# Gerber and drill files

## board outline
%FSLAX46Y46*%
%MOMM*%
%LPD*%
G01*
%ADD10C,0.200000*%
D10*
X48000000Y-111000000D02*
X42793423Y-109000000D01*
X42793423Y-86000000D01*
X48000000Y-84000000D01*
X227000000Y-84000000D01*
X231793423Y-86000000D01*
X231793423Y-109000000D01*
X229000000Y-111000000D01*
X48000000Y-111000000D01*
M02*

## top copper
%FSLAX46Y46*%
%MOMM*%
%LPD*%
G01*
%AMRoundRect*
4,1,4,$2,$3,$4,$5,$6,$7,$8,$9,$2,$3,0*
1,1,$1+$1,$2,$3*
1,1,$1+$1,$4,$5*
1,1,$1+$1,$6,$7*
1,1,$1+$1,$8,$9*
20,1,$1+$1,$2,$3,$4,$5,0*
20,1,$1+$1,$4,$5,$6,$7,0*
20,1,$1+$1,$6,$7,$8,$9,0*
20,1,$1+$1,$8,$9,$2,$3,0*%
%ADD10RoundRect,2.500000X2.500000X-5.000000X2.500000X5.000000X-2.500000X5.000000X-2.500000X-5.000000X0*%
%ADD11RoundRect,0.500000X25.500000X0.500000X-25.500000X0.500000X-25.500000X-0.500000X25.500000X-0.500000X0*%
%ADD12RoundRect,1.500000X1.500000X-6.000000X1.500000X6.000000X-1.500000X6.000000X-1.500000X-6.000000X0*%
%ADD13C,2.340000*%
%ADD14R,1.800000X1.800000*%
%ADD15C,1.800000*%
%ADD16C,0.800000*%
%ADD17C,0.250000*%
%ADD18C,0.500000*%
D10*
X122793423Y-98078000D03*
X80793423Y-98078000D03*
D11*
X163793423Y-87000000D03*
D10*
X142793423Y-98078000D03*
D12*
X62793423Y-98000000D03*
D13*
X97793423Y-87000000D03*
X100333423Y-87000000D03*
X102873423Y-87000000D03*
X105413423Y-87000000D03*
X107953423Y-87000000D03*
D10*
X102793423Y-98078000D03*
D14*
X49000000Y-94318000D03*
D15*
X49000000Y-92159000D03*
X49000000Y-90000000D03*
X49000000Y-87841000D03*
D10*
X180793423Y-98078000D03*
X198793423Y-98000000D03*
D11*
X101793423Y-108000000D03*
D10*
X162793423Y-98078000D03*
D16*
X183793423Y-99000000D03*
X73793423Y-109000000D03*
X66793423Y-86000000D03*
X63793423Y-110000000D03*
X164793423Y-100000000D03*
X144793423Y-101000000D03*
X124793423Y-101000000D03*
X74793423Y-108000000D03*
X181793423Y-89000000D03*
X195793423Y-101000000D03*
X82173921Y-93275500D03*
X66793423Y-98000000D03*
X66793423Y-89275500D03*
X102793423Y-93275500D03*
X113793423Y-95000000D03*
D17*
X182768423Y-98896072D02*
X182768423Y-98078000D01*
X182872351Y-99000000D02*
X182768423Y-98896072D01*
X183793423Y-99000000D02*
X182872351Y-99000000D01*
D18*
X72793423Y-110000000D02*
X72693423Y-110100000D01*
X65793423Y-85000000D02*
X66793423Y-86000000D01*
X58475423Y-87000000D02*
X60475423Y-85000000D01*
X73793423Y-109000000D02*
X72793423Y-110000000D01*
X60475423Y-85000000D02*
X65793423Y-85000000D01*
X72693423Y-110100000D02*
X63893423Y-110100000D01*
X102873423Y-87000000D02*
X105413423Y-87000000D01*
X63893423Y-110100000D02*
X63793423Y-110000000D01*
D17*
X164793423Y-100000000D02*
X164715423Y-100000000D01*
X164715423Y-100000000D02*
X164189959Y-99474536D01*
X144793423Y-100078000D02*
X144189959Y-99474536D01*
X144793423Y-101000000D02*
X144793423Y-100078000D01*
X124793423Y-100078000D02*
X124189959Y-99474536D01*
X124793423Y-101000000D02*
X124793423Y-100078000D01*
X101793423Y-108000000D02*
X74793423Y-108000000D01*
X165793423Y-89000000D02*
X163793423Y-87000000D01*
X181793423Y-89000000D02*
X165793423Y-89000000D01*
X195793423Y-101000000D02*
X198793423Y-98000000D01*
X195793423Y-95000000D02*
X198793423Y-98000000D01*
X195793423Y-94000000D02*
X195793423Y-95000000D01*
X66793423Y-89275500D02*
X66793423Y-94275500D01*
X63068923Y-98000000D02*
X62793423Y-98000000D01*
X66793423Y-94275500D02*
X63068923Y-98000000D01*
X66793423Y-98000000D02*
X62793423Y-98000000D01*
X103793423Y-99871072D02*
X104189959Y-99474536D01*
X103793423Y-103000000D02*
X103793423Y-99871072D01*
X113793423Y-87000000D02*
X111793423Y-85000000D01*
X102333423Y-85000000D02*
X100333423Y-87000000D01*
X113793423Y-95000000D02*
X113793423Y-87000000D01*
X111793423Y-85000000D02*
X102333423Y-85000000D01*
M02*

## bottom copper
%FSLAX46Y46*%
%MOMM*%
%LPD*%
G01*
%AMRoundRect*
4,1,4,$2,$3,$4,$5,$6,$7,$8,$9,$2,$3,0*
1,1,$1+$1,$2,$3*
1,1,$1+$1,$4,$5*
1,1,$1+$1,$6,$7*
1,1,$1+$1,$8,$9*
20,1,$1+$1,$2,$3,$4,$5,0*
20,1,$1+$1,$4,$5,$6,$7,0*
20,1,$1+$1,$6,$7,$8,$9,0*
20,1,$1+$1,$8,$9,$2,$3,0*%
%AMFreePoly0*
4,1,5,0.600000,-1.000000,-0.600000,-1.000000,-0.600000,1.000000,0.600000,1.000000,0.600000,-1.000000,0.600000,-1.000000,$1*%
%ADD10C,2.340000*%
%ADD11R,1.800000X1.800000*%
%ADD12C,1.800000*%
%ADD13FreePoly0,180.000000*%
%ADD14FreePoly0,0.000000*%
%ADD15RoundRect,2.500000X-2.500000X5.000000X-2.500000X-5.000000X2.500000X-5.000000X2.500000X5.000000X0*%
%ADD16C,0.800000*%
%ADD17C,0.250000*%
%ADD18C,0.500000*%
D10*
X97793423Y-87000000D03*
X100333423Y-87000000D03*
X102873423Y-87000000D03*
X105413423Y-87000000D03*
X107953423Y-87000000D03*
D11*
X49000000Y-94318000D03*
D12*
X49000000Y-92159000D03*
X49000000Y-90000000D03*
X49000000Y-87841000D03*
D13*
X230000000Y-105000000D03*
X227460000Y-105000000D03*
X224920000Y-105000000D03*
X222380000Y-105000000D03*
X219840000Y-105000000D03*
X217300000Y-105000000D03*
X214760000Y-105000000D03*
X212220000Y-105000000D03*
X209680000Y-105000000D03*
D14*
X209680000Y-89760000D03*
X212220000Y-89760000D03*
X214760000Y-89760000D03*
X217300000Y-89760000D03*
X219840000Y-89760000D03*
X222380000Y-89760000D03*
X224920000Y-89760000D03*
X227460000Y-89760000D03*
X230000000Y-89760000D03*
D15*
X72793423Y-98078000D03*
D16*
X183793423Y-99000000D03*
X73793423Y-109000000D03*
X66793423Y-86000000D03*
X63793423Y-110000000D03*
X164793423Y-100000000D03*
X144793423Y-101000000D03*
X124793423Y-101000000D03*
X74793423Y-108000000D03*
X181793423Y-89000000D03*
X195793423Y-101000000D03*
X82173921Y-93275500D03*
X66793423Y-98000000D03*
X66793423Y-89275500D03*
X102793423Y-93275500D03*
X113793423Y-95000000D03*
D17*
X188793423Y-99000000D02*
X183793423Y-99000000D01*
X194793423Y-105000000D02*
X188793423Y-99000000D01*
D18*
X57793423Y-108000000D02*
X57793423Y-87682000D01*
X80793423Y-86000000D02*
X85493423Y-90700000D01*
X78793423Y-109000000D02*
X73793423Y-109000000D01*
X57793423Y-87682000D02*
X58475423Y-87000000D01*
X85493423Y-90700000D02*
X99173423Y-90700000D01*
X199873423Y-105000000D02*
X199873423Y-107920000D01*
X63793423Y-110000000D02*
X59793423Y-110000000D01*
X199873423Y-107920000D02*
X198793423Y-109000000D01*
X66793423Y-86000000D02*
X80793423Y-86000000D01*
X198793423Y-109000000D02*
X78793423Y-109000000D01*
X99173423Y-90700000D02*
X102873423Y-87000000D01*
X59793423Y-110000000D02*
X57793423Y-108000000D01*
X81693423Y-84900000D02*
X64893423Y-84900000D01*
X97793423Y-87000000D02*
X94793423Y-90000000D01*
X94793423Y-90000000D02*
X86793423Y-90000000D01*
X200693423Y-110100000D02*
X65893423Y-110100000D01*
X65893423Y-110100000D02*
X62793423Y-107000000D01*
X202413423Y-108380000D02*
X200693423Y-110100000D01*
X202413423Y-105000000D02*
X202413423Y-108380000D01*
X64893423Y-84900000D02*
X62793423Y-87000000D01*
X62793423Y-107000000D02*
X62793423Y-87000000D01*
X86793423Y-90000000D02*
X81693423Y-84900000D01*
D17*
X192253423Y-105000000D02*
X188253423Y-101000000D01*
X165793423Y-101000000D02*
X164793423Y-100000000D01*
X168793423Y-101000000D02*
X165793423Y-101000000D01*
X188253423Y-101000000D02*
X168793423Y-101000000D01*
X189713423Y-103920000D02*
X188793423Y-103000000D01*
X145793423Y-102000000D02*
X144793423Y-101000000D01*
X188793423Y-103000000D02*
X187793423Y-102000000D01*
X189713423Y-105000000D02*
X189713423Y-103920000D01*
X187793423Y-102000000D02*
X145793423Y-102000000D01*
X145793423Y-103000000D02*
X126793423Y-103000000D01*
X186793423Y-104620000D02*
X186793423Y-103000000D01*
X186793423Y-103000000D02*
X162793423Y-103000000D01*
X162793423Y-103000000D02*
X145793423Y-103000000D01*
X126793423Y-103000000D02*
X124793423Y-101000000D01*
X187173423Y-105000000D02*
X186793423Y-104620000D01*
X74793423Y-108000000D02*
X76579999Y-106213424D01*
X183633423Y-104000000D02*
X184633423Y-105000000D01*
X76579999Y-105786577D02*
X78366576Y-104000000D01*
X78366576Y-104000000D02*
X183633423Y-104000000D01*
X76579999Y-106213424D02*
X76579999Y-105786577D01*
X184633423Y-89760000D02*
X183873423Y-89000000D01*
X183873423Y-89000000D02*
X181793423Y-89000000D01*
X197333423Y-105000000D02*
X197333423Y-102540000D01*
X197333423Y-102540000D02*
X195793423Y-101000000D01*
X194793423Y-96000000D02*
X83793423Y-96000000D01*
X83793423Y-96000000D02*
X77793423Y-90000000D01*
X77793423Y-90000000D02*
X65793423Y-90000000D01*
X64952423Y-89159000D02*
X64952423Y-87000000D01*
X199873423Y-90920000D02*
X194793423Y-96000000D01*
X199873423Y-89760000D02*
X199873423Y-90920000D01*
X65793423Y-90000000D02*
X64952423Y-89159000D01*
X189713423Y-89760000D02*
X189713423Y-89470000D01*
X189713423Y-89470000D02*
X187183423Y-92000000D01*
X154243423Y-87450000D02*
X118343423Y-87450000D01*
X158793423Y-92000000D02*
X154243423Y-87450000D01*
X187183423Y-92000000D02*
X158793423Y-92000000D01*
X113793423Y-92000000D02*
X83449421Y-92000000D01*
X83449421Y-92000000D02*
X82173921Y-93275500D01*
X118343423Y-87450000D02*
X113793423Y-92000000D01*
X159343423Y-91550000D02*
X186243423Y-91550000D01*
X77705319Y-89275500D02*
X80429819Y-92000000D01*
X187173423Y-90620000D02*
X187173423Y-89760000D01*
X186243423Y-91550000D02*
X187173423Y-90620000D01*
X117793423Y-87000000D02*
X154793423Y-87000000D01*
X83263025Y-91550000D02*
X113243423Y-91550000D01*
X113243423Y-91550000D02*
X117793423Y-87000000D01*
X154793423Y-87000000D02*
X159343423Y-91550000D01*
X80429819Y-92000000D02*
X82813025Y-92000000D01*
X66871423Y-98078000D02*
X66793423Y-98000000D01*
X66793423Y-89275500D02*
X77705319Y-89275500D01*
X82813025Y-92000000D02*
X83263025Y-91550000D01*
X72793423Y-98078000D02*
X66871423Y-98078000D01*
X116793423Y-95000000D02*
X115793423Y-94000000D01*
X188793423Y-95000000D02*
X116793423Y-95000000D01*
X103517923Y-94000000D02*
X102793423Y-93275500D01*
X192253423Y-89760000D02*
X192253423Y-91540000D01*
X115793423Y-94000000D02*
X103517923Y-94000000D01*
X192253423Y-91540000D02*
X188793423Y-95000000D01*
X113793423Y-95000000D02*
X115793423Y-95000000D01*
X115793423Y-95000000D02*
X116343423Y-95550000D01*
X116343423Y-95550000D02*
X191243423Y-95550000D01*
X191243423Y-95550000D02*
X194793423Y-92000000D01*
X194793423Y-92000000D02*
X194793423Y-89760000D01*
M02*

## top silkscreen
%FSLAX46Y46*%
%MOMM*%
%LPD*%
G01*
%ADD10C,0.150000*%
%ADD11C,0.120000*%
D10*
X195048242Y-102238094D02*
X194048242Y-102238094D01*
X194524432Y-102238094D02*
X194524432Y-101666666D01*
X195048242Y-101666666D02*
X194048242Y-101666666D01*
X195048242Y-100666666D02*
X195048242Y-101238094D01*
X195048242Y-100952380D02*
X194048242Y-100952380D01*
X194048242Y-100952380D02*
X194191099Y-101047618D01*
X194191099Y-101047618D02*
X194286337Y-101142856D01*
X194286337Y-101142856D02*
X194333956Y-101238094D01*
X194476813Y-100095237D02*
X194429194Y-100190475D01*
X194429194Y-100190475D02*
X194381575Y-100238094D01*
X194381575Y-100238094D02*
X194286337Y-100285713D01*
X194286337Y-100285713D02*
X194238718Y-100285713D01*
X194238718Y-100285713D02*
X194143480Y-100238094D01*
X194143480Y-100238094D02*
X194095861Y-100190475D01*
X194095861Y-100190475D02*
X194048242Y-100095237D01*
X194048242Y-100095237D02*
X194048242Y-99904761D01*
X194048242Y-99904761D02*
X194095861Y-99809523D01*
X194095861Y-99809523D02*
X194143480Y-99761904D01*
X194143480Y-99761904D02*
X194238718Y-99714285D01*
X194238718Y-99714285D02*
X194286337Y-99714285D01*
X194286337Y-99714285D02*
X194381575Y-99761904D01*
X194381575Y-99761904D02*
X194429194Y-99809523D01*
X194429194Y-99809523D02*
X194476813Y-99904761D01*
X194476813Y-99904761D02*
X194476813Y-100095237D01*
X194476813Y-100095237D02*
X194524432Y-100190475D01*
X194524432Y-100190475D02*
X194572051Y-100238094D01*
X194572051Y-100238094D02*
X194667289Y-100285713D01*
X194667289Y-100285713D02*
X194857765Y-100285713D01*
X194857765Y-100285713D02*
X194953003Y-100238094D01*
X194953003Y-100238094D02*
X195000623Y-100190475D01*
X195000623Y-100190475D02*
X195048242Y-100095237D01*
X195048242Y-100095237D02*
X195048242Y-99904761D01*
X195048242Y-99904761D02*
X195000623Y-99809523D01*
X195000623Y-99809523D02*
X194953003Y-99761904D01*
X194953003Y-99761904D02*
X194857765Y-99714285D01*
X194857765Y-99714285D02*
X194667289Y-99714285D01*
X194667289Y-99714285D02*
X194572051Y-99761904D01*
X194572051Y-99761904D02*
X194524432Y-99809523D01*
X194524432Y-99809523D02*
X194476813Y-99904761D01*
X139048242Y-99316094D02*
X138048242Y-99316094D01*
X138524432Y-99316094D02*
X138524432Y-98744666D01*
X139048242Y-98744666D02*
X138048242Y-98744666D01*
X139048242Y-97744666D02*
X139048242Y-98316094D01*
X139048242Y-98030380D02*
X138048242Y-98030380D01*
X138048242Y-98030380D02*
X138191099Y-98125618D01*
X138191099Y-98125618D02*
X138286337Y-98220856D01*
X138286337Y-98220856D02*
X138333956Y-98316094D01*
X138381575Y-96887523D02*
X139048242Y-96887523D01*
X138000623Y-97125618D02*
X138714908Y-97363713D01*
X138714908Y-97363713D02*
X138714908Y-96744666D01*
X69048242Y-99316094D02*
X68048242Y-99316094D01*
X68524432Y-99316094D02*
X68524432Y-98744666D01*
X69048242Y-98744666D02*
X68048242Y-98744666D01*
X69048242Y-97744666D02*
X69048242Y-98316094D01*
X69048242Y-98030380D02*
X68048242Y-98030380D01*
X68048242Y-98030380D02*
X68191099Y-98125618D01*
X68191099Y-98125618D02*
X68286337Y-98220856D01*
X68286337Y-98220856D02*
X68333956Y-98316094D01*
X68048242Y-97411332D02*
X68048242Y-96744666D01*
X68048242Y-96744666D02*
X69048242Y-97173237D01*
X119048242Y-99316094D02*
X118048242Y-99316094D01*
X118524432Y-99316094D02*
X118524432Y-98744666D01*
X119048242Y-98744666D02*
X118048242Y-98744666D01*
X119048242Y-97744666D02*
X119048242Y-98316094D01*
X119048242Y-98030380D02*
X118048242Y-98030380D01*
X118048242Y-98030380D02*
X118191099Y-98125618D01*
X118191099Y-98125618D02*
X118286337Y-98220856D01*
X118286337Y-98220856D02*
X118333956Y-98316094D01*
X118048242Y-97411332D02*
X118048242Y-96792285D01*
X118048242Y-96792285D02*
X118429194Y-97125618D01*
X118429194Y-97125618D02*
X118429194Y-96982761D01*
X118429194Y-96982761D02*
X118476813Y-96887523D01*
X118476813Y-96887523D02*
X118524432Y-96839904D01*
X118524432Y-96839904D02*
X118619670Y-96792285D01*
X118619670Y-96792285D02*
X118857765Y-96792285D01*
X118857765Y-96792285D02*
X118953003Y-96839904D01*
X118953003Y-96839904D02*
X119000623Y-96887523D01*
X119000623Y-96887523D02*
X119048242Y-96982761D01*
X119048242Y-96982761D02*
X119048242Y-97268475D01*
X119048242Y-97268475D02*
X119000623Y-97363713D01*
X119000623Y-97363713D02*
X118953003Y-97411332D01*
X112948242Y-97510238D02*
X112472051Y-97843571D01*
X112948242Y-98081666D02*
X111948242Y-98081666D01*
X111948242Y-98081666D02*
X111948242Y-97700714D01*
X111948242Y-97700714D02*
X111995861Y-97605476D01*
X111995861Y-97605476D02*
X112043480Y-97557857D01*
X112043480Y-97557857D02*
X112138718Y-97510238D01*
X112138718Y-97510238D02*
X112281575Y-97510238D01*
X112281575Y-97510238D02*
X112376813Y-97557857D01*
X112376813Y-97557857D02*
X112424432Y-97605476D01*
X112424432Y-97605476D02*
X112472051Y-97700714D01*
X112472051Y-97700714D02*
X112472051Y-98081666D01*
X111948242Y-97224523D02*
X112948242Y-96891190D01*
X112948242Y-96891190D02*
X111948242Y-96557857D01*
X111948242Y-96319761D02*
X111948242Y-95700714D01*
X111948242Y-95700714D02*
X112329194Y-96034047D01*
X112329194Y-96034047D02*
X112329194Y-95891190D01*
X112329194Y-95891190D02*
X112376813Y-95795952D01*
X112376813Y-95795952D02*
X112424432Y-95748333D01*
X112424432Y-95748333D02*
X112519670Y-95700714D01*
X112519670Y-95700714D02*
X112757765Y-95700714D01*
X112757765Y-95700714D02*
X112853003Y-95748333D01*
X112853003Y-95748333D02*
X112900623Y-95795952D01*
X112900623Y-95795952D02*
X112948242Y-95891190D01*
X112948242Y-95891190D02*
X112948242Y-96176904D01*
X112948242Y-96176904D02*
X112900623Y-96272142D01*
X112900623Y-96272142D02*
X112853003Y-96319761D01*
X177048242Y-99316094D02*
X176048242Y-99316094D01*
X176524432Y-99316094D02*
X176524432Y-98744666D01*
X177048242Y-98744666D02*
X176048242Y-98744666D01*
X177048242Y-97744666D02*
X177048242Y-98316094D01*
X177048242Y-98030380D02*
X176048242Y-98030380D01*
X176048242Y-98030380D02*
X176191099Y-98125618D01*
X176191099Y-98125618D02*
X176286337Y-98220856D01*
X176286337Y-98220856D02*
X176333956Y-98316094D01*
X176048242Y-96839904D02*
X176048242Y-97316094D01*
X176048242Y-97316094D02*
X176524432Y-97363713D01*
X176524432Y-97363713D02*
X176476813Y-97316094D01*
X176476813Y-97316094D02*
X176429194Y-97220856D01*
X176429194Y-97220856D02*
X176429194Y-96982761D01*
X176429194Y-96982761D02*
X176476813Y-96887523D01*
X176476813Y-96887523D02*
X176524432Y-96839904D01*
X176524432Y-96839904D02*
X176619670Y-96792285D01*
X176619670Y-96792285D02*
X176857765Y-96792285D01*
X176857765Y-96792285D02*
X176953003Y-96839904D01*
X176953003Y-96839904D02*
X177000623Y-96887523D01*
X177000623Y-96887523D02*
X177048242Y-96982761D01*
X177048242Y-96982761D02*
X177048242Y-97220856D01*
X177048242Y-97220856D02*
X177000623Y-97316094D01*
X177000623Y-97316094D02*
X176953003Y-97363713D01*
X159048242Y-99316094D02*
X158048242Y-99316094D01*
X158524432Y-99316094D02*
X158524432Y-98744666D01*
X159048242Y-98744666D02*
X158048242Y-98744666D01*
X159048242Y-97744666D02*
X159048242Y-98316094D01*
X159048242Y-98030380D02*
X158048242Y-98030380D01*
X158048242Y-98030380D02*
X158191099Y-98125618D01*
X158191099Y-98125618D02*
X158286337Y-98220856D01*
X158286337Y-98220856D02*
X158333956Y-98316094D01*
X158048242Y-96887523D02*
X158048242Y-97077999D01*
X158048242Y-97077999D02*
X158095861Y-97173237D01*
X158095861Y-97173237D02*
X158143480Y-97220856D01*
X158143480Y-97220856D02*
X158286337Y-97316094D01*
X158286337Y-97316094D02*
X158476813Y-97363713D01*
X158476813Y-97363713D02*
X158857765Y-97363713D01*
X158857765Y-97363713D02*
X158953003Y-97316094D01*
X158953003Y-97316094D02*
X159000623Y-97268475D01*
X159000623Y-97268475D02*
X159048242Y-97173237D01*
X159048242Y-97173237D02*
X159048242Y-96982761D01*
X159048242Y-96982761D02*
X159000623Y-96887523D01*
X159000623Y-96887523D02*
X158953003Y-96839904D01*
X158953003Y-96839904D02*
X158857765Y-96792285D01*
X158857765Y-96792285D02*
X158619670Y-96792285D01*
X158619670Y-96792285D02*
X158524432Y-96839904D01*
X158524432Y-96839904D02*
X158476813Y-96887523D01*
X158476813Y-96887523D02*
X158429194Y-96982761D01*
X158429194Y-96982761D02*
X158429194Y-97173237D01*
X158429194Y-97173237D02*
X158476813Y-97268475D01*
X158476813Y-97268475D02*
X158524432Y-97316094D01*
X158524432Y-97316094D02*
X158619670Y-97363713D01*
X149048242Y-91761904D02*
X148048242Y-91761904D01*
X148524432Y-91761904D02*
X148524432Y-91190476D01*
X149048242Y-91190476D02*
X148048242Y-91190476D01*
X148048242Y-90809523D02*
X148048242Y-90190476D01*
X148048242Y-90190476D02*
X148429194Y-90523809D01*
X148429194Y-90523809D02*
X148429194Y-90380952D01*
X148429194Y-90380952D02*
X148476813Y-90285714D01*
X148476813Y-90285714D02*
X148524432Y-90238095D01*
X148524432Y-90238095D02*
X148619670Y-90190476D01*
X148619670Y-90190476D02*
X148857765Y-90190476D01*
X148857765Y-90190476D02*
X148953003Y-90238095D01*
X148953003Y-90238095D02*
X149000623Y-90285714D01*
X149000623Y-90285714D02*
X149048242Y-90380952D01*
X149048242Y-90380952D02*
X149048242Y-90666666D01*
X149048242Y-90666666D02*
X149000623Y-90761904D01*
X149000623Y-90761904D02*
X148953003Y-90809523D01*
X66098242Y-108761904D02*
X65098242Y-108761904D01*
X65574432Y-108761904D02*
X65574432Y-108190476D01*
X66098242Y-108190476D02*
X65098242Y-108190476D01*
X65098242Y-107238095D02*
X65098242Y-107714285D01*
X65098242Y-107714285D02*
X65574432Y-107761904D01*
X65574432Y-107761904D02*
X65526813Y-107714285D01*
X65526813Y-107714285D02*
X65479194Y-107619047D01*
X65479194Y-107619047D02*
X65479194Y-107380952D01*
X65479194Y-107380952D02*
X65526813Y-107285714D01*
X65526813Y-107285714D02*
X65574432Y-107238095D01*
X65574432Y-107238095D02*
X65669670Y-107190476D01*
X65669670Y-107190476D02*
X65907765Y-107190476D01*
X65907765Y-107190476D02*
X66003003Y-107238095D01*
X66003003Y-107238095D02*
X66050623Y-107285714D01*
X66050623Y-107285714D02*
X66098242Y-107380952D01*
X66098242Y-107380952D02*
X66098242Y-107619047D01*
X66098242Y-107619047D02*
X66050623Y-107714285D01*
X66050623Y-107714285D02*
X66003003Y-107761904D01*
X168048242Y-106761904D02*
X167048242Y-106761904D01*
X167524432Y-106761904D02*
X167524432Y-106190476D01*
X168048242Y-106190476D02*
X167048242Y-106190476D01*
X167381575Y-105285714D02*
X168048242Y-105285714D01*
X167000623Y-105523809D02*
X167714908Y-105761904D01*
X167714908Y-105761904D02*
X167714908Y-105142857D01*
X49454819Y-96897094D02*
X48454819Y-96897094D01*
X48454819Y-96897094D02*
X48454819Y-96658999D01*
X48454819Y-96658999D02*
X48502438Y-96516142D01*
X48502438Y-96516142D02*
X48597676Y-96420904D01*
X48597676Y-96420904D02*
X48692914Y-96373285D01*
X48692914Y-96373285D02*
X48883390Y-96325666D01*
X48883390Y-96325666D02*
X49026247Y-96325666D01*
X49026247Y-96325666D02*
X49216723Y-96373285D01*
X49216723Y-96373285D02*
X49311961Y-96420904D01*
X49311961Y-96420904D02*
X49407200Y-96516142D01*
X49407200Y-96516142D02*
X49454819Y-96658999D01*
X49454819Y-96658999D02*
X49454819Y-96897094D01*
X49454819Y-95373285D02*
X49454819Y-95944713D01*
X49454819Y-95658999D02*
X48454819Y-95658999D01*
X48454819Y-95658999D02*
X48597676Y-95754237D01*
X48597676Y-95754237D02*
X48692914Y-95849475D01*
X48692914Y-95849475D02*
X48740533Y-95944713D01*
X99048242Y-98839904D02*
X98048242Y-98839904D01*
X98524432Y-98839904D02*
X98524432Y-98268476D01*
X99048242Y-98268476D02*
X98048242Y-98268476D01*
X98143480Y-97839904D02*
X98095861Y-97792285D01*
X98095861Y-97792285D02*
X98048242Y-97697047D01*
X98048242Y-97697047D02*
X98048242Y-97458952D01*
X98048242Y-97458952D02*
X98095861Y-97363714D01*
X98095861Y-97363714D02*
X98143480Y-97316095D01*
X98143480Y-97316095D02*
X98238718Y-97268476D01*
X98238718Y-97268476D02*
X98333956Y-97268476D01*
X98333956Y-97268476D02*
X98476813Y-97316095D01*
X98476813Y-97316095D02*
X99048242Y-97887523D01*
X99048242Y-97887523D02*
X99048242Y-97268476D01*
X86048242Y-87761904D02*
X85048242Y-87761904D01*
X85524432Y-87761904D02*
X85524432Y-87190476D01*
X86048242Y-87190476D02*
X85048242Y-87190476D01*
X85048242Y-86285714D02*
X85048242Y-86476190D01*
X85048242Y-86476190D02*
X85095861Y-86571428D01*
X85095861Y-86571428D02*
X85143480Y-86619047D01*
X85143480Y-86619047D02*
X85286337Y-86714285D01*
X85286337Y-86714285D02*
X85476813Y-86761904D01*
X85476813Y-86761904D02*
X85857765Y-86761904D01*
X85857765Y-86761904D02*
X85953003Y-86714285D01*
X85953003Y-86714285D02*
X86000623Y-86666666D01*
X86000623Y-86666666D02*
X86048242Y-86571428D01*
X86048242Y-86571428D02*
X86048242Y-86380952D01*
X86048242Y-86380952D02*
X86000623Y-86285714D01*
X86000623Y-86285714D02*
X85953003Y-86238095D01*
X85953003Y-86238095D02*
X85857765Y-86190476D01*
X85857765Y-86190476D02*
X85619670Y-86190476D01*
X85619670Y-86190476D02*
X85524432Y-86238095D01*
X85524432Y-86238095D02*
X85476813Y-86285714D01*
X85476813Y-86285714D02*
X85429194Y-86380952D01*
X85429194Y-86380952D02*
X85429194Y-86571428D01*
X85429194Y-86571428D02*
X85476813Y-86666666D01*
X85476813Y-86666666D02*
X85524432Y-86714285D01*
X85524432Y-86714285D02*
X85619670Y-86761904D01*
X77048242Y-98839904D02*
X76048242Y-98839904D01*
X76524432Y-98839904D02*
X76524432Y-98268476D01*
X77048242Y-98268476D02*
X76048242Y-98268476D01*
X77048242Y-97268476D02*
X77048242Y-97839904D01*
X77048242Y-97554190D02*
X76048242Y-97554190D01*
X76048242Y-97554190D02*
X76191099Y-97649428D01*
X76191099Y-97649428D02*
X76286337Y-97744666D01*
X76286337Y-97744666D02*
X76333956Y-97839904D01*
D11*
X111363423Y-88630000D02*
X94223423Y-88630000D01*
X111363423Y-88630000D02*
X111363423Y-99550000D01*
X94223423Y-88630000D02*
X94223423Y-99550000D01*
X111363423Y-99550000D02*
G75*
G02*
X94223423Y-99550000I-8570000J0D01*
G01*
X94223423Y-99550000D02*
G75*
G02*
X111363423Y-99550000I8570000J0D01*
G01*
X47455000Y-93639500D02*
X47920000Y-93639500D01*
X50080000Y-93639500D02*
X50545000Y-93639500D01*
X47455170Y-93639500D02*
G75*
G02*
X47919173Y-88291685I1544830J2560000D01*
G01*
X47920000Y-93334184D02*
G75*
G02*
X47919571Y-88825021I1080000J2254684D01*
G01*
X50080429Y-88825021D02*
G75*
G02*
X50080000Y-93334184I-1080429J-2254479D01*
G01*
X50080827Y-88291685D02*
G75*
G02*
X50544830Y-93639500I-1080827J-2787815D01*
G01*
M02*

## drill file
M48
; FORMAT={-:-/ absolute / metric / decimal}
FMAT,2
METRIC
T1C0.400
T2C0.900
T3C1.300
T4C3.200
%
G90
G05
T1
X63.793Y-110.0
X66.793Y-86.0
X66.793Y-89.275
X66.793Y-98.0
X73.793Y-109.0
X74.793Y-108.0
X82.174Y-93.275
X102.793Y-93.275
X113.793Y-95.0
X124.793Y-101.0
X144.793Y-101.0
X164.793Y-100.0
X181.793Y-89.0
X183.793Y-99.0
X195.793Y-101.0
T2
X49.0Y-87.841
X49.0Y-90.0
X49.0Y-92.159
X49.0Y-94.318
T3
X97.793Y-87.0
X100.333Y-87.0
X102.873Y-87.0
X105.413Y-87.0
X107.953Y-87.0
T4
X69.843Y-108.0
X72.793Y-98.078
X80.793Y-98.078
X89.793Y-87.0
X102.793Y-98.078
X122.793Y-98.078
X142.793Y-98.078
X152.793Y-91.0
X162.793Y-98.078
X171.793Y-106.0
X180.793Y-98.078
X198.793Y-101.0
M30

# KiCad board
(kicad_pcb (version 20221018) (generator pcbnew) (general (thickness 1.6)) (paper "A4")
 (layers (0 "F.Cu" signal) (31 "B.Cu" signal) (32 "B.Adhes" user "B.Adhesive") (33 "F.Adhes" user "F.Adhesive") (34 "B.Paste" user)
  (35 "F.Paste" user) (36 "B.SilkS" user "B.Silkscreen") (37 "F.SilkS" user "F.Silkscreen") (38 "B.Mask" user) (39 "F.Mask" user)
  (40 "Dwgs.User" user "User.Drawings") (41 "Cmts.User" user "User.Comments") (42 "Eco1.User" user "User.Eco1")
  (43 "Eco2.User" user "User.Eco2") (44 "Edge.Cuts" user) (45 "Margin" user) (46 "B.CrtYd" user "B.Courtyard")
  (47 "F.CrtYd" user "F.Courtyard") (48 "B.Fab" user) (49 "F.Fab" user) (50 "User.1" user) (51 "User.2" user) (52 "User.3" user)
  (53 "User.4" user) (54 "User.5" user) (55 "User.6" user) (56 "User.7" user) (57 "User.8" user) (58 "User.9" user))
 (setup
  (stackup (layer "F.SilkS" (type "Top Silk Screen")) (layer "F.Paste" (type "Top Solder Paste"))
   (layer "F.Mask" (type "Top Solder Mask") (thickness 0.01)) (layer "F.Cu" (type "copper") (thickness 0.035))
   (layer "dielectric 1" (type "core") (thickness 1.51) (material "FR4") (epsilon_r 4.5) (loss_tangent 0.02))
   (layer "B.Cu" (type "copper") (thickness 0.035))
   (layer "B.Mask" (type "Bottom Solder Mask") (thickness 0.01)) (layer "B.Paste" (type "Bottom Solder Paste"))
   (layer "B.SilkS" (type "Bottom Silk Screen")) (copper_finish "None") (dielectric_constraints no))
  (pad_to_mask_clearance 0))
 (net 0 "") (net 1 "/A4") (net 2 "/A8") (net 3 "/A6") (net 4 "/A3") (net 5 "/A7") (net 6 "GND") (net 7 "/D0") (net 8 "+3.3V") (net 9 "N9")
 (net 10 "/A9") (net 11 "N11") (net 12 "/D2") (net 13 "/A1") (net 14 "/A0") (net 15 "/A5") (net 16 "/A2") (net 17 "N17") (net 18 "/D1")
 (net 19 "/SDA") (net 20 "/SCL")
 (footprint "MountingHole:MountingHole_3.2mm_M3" (layer "F.Cu") (at 198.793423 101 90)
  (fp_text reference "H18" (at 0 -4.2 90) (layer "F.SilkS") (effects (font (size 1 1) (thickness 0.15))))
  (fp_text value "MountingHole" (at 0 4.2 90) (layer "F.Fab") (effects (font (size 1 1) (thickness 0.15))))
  (pad "" np_thru_hole circle (at 0 0 90) (size 3.2 3.2) (drill 3.2) (layers "*.Cu" "*.Mask")))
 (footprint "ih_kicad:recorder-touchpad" (layer "F.Cu") (at 122.793423 98.078 90)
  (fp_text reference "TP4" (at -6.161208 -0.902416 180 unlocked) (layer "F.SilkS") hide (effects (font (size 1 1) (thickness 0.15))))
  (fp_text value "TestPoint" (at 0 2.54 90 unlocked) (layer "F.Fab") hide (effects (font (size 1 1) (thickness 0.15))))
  (pad "1" smd roundrect (at 0 0 90) (size 15 10) (layers "F.Cu" "F.Mask") (roundrect_rratio 0.25) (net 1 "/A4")))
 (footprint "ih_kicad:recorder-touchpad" (layer "F.Cu") (at 80.793423 98.078 90)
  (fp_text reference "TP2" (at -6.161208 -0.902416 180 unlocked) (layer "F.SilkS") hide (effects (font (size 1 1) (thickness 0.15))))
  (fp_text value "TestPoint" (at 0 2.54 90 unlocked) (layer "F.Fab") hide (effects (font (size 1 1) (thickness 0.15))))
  (pad "1" smd roundrect (at 0 0 90) (size 15 10) (layers "F.Cu" "F.Mask") (roundrect_rratio 0.25) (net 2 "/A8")))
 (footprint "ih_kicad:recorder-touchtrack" (layer "F.Cu") (at 163.793423 87 180)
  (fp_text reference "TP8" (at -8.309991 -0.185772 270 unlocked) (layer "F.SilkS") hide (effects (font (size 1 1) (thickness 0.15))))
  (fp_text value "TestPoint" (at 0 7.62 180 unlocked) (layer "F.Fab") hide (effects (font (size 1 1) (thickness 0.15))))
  (pad "1" smd roundrect (at 0 0 180) (size 52 2) (layers "F.Cu" "F.Mask") (roundrect_rratio 0.25) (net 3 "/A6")))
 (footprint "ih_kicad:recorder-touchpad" (layer "F.Cu") (at 142.793423 98.078 90)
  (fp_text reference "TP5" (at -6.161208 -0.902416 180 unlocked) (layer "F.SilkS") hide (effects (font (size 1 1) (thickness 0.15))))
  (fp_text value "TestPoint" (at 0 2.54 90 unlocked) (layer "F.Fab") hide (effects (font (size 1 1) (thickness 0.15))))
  (pad "1" smd roundrect (at 0 0 90) (size 15 10) (layers "F.Cu" "F.Mask") (roundrect_rratio 0.25) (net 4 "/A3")))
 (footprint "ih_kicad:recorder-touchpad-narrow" (layer "F.Cu") (at 62.793423 98 90)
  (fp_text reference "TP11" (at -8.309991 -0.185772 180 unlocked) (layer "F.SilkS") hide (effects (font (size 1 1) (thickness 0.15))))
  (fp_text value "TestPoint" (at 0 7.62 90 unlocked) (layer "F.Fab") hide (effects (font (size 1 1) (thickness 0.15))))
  (pad "1" smd roundrect (at 0 0 90) (size 15 6) (layers "F.Cu" "F.Mask") (roundrect_rratio 0.25) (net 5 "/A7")))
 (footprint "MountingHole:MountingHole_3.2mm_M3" (layer "F.Cu") (at 142.793423 98.078 90)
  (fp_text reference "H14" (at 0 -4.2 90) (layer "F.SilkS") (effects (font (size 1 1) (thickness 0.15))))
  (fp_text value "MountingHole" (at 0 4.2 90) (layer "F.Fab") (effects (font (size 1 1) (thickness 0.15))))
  (pad "" np_thru_hole circle (at 0 0 90) (size 3.2 3.2) (drill 3.2) (layers "*.Cu" "*.Mask")))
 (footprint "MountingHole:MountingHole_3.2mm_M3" (layer "F.Cu") (at 72.793423 98.078 90)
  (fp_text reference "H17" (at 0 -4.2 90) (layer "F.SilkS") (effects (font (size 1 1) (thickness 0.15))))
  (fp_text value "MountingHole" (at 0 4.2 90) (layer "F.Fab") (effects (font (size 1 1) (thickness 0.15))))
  (pad "" np_thru_hole circle (at 0 0 90) (size 3.2 3.2) (drill 3.2) (layers "*.Cu" "*.Mask")))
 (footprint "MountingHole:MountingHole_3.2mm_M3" (layer "F.Cu") (at 122.793423 98.078 90)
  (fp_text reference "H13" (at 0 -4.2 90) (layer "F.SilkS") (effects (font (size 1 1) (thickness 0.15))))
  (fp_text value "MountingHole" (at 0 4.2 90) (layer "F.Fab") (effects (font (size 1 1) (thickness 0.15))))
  (pad "" np_thru_hole circle (at 0 0 90) (size 3.2 3.2) (drill 3.2) (layers "*.Cu" "*.Mask")))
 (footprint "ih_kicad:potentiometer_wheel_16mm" (layer "F.Cu") (at 97.793423 87 -90)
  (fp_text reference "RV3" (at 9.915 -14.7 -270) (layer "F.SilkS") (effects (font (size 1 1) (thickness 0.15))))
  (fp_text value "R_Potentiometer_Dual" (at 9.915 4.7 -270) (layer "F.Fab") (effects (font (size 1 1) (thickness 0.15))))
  (fp_line (start 1.63 -13.57) (end 1.63 3.57) (stroke (width 0.12) (type solid)) (layer "F.SilkS"))
  (fp_line (start 1.63 -13.57) (end 12.55 -13.57) (stroke (width 0.12) (type solid)) (layer "F.SilkS"))
  (fp_line (start 1.63 3.57) (end 12.55 3.57) (stroke (width 0.12) (type solid)) (layer "F.SilkS"))
  (fp_circle (center 12.55 -5) (end 21.12 -5) (stroke (width 0.12) (type solid)) (fill none) (layer "F.SilkS"))
  (pad "1" thru_hole circle (at 0 0 270) (size 2.34 2.34) (drill 1.3) (layers "*.Cu" "*.Mask") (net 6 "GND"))
  (pad "2" thru_hole circle (at 0 -2.54 270) (size 2.34 2.34) (drill 1.3) (layers "*.Cu" "*.Mask") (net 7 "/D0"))
  (pad "3" thru_hole circle (at 0 -5.08 270) (size 2.34 2.34) (drill 1.3) (layers "*.Cu" "*.Mask") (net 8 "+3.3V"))
  (pad "4" thru_hole circle (at 0 -7.62 270) (size 2.34 2.34) (drill 1.3) (layers "*.Cu" "*.Mask") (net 8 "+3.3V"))
  (pad "5" thru_hole circle (at 0 -10.16 270) (size 2.34 2.34) (drill 1.3) (layers "*.Cu" "*.Mask") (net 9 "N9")))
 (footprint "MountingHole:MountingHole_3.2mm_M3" (layer "F.Cu") (at 180.793423 98.078 90)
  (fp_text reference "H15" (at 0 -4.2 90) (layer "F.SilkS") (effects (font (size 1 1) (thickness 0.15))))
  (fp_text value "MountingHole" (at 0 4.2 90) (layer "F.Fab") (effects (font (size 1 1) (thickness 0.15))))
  (pad "" np_thru_hole circle (at 0 0 90) (size 3.2 3.2) (drill 3.2) (layers "*.Cu" "*.Mask")))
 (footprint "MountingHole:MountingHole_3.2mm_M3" (layer "F.Cu") (at 162.793423 98.078 90)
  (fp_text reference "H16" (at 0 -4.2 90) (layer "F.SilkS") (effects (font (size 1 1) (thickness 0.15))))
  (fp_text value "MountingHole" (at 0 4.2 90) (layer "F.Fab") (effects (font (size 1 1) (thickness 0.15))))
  (pad "" np_thru_hole circle (at 0 0 90) (size 3.2 3.2) (drill 3.2) (layers "*.Cu" "*.Mask")))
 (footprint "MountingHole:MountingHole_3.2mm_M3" (layer "F.Cu") (at 152.793423 91 90)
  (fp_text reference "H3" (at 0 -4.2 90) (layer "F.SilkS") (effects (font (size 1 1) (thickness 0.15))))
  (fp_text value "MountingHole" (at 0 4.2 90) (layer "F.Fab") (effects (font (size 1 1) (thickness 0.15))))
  (pad "" np_thru_hole circle (at 0 0 90) (size 3.2 3.2) (drill 3.2) (layers "*.Cu" "*.Mask")))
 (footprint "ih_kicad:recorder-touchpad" (layer "F.Cu") (at 102.793423 98.078 90)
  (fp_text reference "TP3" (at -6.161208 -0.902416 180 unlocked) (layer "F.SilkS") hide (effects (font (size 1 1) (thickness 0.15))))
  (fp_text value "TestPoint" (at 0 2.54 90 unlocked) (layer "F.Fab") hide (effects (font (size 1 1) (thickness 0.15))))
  (pad "1" smd roundrect (at 0 0 90) (size 15 10) (layers "F.Cu" "F.Mask") (roundrect_rratio 0.25) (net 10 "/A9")))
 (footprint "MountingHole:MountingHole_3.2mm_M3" (layer "F.Cu") (at 69.843423 108 90)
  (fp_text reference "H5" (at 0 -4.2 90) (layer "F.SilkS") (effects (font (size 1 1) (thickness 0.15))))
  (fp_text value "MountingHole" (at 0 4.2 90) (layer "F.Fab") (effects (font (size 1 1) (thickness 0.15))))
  (pad "" np_thru_hole circle (at 0 0 90) (size 3.2 3.2) (drill 3.2) (layers "*.Cu" "*.Mask")))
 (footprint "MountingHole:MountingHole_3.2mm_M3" (layer "F.Cu") (at 171.793423 106 90)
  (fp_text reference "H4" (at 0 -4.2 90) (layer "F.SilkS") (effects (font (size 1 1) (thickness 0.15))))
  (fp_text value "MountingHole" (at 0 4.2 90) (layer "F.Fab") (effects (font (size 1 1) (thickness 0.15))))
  (pad "" np_thru_hole circle (at 0 0 90) (size 3.2 3.2) (drill 3.2) (layers "*.Cu" "*.Mask")))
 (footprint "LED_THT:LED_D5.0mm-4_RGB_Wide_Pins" (layer "F.Cu") (at 49 94.318 90)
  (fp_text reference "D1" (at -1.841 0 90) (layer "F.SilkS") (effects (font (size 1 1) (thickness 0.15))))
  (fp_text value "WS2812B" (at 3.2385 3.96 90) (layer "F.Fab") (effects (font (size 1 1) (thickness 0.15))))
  (fp_line (start 0.6785 -1.545) (end 0.6785 -1.08) (stroke (width 0.12) (type solid)) (layer "F.SilkS"))
  (fp_line (start 0.6785 1.08) (end 0.6785 1.545) (stroke (width 0.12) (type solid)) (layer "F.SilkS"))
  (fp_arc (start 0.6785 -1.54483) (mid 3.496956 -2.978809) (end 6.026315 -1.080827) (stroke (width 0.12) (type solid)) (layer "F.SilkS"))
  (fp_arc (start 0.983816 -1.08) (mid 3.238262 -2.5) (end 5.492979 -1.080429) (stroke (width 0.12) (type solid)) (layer "F.SilkS"))
  (fp_arc (start 5.492979 1.080429) (mid 3.238262 2.5) (end 0.983816 1.08) (stroke (width 0.12) (type solid)) (layer "F.SilkS"))
  (fp_arc (start 6.026315 1.080827) (mid 3.496956 2.978808) (end 0.6785 1.54483) (stroke (width 0.12) (type solid)) (layer "F.SilkS"))
  (pad "1" thru_hole rect (at 0 0 90) (size 1.8 1.8) (drill 0.9) (layers "*.Cu" "*.Mask") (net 8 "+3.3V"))
  (pad "2" thru_hole circle (at 2.159 0 90) (size 1.8 1.8) (drill 0.9) (layers "*.Cu" "*.Mask") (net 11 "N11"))
  (pad "3" thru_hole circle (at 4.318 0 90) (size 1.8 1.8) (drill 0.9) (layers "*.Cu" "*.Mask") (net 6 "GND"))
  (pad "4" thru_hole circle (at 6.477 0 90) (size 1.8 1.8) (drill 0.9) (layers "*.Cu" "*.Mask") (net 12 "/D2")))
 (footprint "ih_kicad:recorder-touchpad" (layer "F.Cu") (at 180.793423 98.078 90)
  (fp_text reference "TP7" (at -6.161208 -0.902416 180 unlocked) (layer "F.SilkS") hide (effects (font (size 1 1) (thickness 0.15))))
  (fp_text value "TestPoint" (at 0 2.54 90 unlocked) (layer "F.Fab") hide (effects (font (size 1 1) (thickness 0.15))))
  (pad "1" smd roundrect (at 0 0 90) (size 15 10) (layers "F.Cu" "F.Mask") (roundrect_rratio 0.25) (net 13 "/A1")))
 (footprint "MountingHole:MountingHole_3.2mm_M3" (layer "F.Cu") (at 102.793423 98.078 90)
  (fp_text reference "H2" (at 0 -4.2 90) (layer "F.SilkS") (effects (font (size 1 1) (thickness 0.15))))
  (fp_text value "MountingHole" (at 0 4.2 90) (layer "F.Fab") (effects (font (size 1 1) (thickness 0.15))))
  (pad "" np_thru_hole circle (at 0 0 90) (size 3.2 3.2) (drill 3.2) (layers "*.Cu" "*.Mask")))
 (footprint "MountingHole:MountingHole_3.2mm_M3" (layer "F.Cu") (at 89.793423 87 90)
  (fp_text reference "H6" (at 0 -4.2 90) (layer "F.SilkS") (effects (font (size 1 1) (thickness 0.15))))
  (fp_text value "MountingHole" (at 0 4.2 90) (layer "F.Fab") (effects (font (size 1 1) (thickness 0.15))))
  (pad "" np_thru_hole circle (at 0 0 90) (size 3.2 3.2) (drill 3.2) (layers "*.Cu" "*.Mask")))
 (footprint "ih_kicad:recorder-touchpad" (layer "F.Cu") (at 198.793423 98 90)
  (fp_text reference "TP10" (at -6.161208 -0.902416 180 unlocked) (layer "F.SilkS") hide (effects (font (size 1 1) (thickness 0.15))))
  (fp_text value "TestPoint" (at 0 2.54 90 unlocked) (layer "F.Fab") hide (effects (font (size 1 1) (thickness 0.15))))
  (pad "1" smd roundrect (at 0 0 90) (size 15 10) (layers "F.Cu" "F.Mask") (roundrect_rratio 0.25) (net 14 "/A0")))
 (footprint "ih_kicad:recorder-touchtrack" (layer "F.Cu") (at 101.793423 108 180)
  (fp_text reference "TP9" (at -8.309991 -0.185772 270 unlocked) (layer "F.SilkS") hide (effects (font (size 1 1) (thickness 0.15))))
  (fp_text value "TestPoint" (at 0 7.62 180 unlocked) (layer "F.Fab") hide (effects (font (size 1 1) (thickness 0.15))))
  (pad "1" smd roundrect (at 0 0 180) (size 52 2) (layers "F.Cu" "F.Mask") (roundrect_rratio 0.25) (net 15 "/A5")))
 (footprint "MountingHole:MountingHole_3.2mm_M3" (layer "F.Cu") (at 80.793423 98.078 90)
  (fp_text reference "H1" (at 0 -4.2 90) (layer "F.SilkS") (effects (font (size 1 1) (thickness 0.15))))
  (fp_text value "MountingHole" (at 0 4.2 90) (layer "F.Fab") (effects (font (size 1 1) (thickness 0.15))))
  (pad "" np_thru_hole circle (at 0 0 90) (size 3.2 3.2) (drill 3.2) (layers "*.Cu" "*.Mask")))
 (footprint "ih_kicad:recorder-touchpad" (layer "F.Cu") (at 162.793423 98.078 90)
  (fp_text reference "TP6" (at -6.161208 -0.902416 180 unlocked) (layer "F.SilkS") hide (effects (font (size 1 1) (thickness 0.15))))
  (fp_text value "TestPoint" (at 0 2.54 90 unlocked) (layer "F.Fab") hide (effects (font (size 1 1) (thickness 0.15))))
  (pad "1" smd roundrect (at 0 0 90) (size 15 10) (layers "F.Cu" "F.Mask") (roundrect_rratio 0.25) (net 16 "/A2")))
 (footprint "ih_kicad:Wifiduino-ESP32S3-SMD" (layer "B.Cu") (at 219.84 97.38 90)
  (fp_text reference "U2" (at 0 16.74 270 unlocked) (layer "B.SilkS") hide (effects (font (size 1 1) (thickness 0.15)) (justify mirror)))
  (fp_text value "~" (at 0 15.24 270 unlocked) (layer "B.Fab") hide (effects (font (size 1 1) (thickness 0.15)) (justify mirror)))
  (pad "1" smd custom (at -7.62 10.16 180) (size 1.2 2) (layers "B.Cu" "B.Paste" "B.Mask") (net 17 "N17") (thermal_bridge_angle 45)
   (options (clearance outline) (anchor rect)) (primitives))
  (pad "2" smd custom (at -7.62 7.62 180) (size 1.2 2) (layers "B.Cu" "B.Paste" "B.Mask") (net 6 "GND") (thermal_bridge_angle 45)
   (options (clearance outline) (anchor rect)) (primitives))
  (pad "3" smd custom (at -7.62 5.08 180) (size 1.2 2) (layers "B.Cu" "B.Paste" "B.Mask") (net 8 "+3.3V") (thermal_bridge_angle 45)
   (options (clearance outline) (anchor rect)) (primitives))
  (pad "4" smd custom (at -7.62 2.54 180) (size 1.2 2) (layers "B.Cu" "B.Paste" "B.Mask") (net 14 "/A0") (thermal_bridge_angle 45)
   (options (clearance outline) (anchor rect)) (primitives))
  (pad "5" smd custom (at -7.62 0 180) (size 1.2 2) (layers "B.Cu" "B.Paste" "B.Mask") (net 13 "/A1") (thermal_bridge_angle 45)
   (options (clearance outline) (anchor rect)) (primitives))
  (pad "6" smd custom (at -7.62 -2.54 180) (size 1.2 2) (layers "B.Cu" "B.Paste" "B.Mask") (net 16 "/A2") (thermal_bridge_angle 45)
   (options (clearance outline) (anchor rect)) (primitives))
  (pad "7" smd custom (at -7.62 -5.08 180) (size 1.2 2) (layers "B.Cu" "B.Paste" "B.Mask") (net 4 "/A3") (thermal_bridge_angle 45)
   (options (clearance outline) (anchor rect)) (primitives))
  (pad "8" smd custom (at -7.62 -7.62 180) (size 1.2 2) (layers "B.Cu" "B.Paste" "B.Mask") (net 1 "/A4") (thermal_bridge_angle 45)
   (options (clearance outline) (anchor rect)) (primitives))
  (pad "9" smd custom (at -7.62 -10.16 180) (size 1.2 2) (layers "B.Cu" "B.Paste" "B.Mask") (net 15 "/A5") (thermal_bridge_angle 45)
   (options (clearance outline) (anchor rect)) (primitives))
  (pad "10" smd custom (at 7.62 -10.16) (size 1.2 2) (layers "B.Cu" "B.Paste" "B.Mask") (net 3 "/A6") (thermal_bridge_angle 45)
   (options (clearance outline) (anchor rect)) (primitives))
  (pad "11" smd custom (at 7.62 -7.62) (size 1.2 2) (layers "B.Cu" "B.Paste" "B.Mask") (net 5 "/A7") (thermal_bridge_angle 45)
   (options (clearance outline) (anchor rect)) (primitives))
  (pad "12" smd custom (at 7.62 -5.08) (size 1.2 2) (layers "B.Cu" "B.Paste" "B.Mask") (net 2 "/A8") (thermal_bridge_angle 45)
   (options (clearance outline) (anchor rect)) (primitives))
  (pad "13" smd custom (at 7.62 -2.54) (size 1.2 2) (layers "B.Cu" "B.Paste" "B.Mask") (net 10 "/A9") (thermal_bridge_angle 45)
   (options (clearance outline) (anchor rect)) (primitives))
  (pad "14" smd custom (at 7.62 0) (size 1.2 2) (layers "B.Cu" "B.Paste" "B.Mask") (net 7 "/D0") (thermal_bridge_angle 45)
   (options (clearance outline) (anchor rect)) (primitives))
  (pad "15" smd custom (at 7.62 2.54) (size 1.2 2) (layers "B.Cu" "B.Paste" "B.Mask") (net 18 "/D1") (thermal_bridge_angle 45)
   (options (clearance outline) (anchor rect)) (primitives))
  (pad "16" smd custom (at 7.62 5.08) (size 1.2 2) (layers "B.Cu" "B.Paste" "B.Mask") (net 12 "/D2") (thermal_bridge_angle 45)
   (options (clearance outline) (anchor rect)) (primitives))
  (pad "17" smd custom (at 7.62 7.62) (size 1.2 2) (layers "B.Cu" "B.Paste" "B.Mask") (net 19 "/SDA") (thermal_bridge_angle 45)
   (options (clearance outline) (anchor rect)) (primitives))
  (pad "18" smd custom (at 7.62 10.16) (size 1.2 2) (layers "B.Cu" "B.Paste" "B.Mask") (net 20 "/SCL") (thermal_bridge_angle 45)
   (options (clearance outline) (anchor rect)) (primitives)))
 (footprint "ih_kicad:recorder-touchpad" (layer "B.Cu") (at 72.793423 98.078 -90)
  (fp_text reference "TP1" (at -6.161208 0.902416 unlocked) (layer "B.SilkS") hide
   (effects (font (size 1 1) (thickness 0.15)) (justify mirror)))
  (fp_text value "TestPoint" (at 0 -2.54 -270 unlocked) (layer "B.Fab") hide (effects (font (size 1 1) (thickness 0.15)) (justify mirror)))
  (pad "1" smd roundrect (at 0 0 270) (size 15 10) (layers "B.Cu" "B.Mask") (roundrect_rratio 0.25) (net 5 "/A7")))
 (gr_poly
  (pts (xy 48 111) (xy 42.793423 109) (xy 42.793423 86) (xy 48 84) (xy 227 84) (xy 231.793423 86) (xy 231.793423 109) (xy 229 111))
  (stroke (width 0.2) (type solid)) (fill none) (layer "Edge.Cuts"))
 (segment (start 182.768423 98.896072) (end 182.768423 98.078) (width 0.25) (layer "F.Cu") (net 13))
 (segment (start 182.872351 99) (end 182.768423 98.896072) (width 0.25) (layer "F.Cu") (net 13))
 (segment (start 183.793423 99) (end 182.872351 99) (width 0.25) (layer "F.Cu") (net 13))
 (via (at 183.793423 99) (size 0.8) (drill 0.4) (layers "F.Cu" "B.Cu") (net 13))
 (segment (start 188.793423 99) (end 183.793423 99) (width 0.25) (layer "B.Cu") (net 13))
 (segment (start 194.793423 105) (end 188.793423 99) (width 0.25) (layer "B.Cu") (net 13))
 (segment (start 72.793423 110) (end 72.693423 110.1) (width 0.5) (layer "F.Cu") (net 8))
 (segment (start 65.793423 85) (end 66.793423 86) (width 0.5) (layer "F.Cu") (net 8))
 (segment (start 58.475423 87) (end 60.475423 85) (width 0.5) (layer "F.Cu") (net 8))
 (segment (start 73.793423 109) (end 72.793423 110) (width 0.5) (layer "F.Cu") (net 8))
 (segment (start 60.475423 85) (end 65.793423 85) (width 0.5) (layer "F.Cu") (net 8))
 (segment (start 72.693423 110.1) (end 63.893423 110.1) (width 0.5) (layer "F.Cu") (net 8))
 (segment (start 102.873423 87) (end 105.413423 87) (width 0.5) (layer "F.Cu") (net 8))
 (segment (start 63.893423 110.1) (end 63.793423 110) (width 0.5) (layer "F.Cu") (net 8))
 (via (at 73.793423 109) (size 0.8) (drill 0.4) (layers "F.Cu" "B.Cu") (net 8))
 (via (at 66.793423 86) (size 0.8) (drill 0.4) (layers "F.Cu" "B.Cu") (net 8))
 (via (at 63.793423 110) (size 0.8) (drill 0.4) (layers "F.Cu" "B.Cu") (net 8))
 (segment (start 57.793423 108) (end 57.793423 87.682) (width 0.5) (layer "B.Cu") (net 8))
 (segment (start 80.793423 86) (end 85.493423 90.7) (width 0.5) (layer "B.Cu") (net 8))
 (segment (start 78.793423 109) (end 73.793423 109) (width 0.5) (layer "B.Cu") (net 8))
 (segment (start 57.793423 87.682) (end 58.475423 87) (width 0.5) (layer "B.Cu") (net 8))
 (segment (start 85.493423 90.7) (end 99.173423 90.7) (width 0.5) (layer "B.Cu") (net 8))
 (segment (start 199.873423 105) (end 199.873423 107.92) (width 0.5) (layer "B.Cu") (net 8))
 (segment (start 63.793423 110) (end 59.793423 110) (width 0.5) (layer "B.Cu") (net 8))
 (segment (start 199.873423 107.92) (end 198.793423 109) (width 0.5) (layer "B.Cu") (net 8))
 (segment (start 66.793423 86) (end 80.793423 86) (width 0.5) (layer "B.Cu") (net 8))
 (segment (start 198.793423 109) (end 78.793423 109) (width 0.5) (layer "B.Cu") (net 8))
 (segment (start 99.173423 90.7) (end 102.873423 87) (width 0.5) (layer "B.Cu") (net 8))
 (segment (start 59.793423 110) (end 57.793423 108) (width 0.5) (layer "B.Cu") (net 8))
 (segment (start 81.693423 84.9) (end 64.893423 84.9) (width 0.5) (layer "B.Cu") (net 6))
 (segment (start 97.793423 87) (end 94.793423 90) (width 0.5) (layer "B.Cu") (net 6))
 (segment (start 94.793423 90) (end 86.793423 90) (width 0.5) (layer "B.Cu") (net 6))
 (segment (start 200.693423 110.1) (end 65.893423 110.1) (width 0.5) (layer "B.Cu") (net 6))
 (segment (start 65.893423 110.1) (end 62.793423 107) (width 0.5) (layer "B.Cu") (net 6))
 (segment (start 202.413423 108.38) (end 200.693423 110.1) (width 0.5) (layer "B.Cu") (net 6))
 (segment (start 202.413423 105) (end 202.413423 108.38) (width 0.5) (layer "B.Cu") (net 6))
 (segment (start 64.893423 84.9) (end 62.793423 87) (width 0.5) (layer "B.Cu") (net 6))
 (segment (start 62.793423 107) (end 62.793423 87) (width 0.5) (layer "B.Cu") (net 6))
 (segment (start 86.793423 90) (end 81.693423 84.9) (width 0.5) (layer "B.Cu") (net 6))
 (segment (start 164.793423 100) (end 164.715423 100) (width 0.25) (layer "F.Cu") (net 16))
 (segment (start 164.715423 100) (end 164.189959 99.474536) (width 0.25) (layer "F.Cu") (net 16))
 (via (at 164.793423 100) (size 0.8) (drill 0.4) (layers "F.Cu" "B.Cu") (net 16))
 (segment (start 192.253423 105) (end 188.253423 101) (width 0.25) (layer "B.Cu") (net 16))
 (segment (start 165.793423 101) (end 164.793423 100) (width 0.25) (layer "B.Cu") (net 16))
 (segment (start 168.793423 101) (end 165.793423 101) (width 0.25) (layer "B.Cu") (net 16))
 (segment (start 188.253423 101) (end 168.793423 101) (width 0.25) (layer "B.Cu") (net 16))
 (segment (start 144.793423 100.078) (end 144.189959 99.474536) (width 0.25) (layer "F.Cu") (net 4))
 (segment (start 144.793423 101) (end 144.793423 100.078) (width 0.25) (layer "F.Cu") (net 4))
 (via (at 144.793423 101) (size 0.8) (drill 0.4) (layers "F.Cu" "B.Cu") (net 4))
 (segment (start 189.713423 103.92) (end 188.793423 103) (width 0.25) (layer "B.Cu") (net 4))
 (segment (start 145.793423 102) (end 144.793423 101) (width 0.25) (layer "B.Cu") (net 4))
 (segment (start 188.793423 103) (end 187.793423 102) (width 0.25) (layer "B.Cu") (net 4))
 (segment (start 189.713423 105) (end 189.713423 103.92) (width 0.25) (layer "B.Cu") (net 4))
 (segment (start 187.793423 102) (end 145.793423 102) (width 0.25) (layer "B.Cu") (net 4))
 (segment (start 124.793423 100.078) (end 124.189959 99.474536) (width 0.25) (layer "F.Cu") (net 1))
 (segment (start 124.793423 101) (end 124.793423 100.078) (width 0.25) (layer "F.Cu") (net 1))
 (via (at 124.793423 101) (size 0.8) (drill 0.4) (layers "F.Cu" "B.Cu") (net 1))
 (segment (start 145.793423 103) (end 126.793423 103) (width 0.25) (layer "B.Cu") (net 1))
 (segment (start 186.793423 104.62) (end 186.793423 103) (width 0.25) (layer "B.Cu") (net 1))
 (segment (start 186.793423 103) (end 162.793423 103) (width 0.25) (layer "B.Cu") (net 1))
 (segment (start 162.793423 103) (end 145.793423 103) (width 0.25) (layer "B.Cu") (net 1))
 (segment (start 126.793423 103) (end 124.793423 101) (width 0.25) (layer "B.Cu") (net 1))
 (segment (start 187.173423 105) (end 186.793423 104.62) (width 0.25) (layer "B.Cu") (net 1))
 (segment (start 101.793423 108) (end 74.793423 108) (width 0.25) (layer "F.Cu") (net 15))
 (via (at 74.793423 108) (size 0.8) (drill 0.4) (layers "F.Cu" "B.Cu") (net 15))
 (segment (start 74.793423 108) (end 76.579999 106.213424) (width 0.25) (layer "B.Cu") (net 15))
 (segment (start 183.633423 104) (end 184.633423 105) (width 0.25) (layer "B.Cu") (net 15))
 (segment (start 76.579999 105.786577) (end 78.366576 104) (width 0.25) (layer "B.Cu") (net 15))
 (segment (start 78.366576 104) (end 183.633423 104) (width 0.25) (layer "B.Cu") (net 15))
 (segment (start 76.579999 106.213424) (end 76.579999 105.786577) (width 0.25) (layer "B.Cu") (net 15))
 (segment (start 165.793423 89) (end 163.793423 87) (width 0.25) (layer "F.Cu") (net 3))
 (segment (start 181.793423 89) (end 165.793423 89) (width 0.25) (layer "F.Cu") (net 3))
 (via (at 181.793423 89) (size 0.8) (drill 0.4) (layers "F.Cu" "B.Cu") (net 3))
 (segment (start 184.633423 89.76) (end 183.873423 89) (width 0.25) (layer "B.Cu") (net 3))
 (segment (start 183.873423 89) (end 181.793423 89) (width 0.25) (layer "B.Cu") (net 3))
 (segment (start 195.793423 101) (end 198.793423 98) (width 0.25) (layer "F.Cu") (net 14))
 (segment (start 195.793423 95) (end 198.793423 98) (width 0.25) (layer "F.Cu") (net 14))
 (segment (start 195.793423 94) (end 195.793423 95) (width 0.25) (layer "F.Cu") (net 14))
 (via (at 195.793423 101) (size 0.8) (drill 0.4) (layers "F.Cu" "B.Cu") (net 14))
 (segment (start 197.333423 105) (end 197.333423 102.54) (width 0.25) (layer "B.Cu") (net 14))
 (segment (start 197.333423 102.54) (end 195.793423 101) (width 0.25) (layer "B.Cu") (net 14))
 (segment (start 194.793423 96) (end 83.793423 96) (width 0.25) (layer "B.Cu") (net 12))
 (segment (start 83.793423 96) (end 77.793423 90) (width 0.25) (layer "B.Cu") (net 12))
 (segment (start 77.793423 90) (end 65.793423 90) (width 0.25) (layer "B.Cu") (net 12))
 (segment (start 64.952423 89.159) (end 64.952423 87) (width 0.25) (layer "B.Cu") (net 12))
 (segment (start 199.873423 90.92) (end 194.793423 96) (width 0.25) (layer "B.Cu") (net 12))
 (segment (start 199.873423 89.76) (end 199.873423 90.92) (width 0.25) (layer "B.Cu") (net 12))
 (segment (start 65.793423 90) (end 64.952423 89.159) (width 0.25) (layer "B.Cu") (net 12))
 (via (at 82.173921 93.2755) (size 0.8) (drill 0.4) (layers "F.Cu" "B.Cu") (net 2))
 (segment (start 189.713423 89.76) (end 189.713423 89.47) (width 0.25) (layer "B.Cu") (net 2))
 (segment (start 189.713423 89.47) (end 187.183423 92) (width 0.25) (layer "B.Cu") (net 2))
 (segment (start 154.243423 87.45) (end 118.343423 87.45) (width 0.25) (layer "B.Cu") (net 2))
 (segment (start 158.793423 92) (end 154.243423 87.45) (width 0.25) (layer "B.Cu") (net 2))
 (segment (start 187.183423 92) (end 158.793423 92) (width 0.25) (layer "B.Cu") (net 2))
 (segment (start 113.793423 92) (end 83.449421 92) (width 0.25) (layer "B.Cu") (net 2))
 (segment (start 83.449421 92) (end 82.173921 93.2755) (width 0.25) (layer "B.Cu") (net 2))
 (segment (start 118.343423 87.45) (end 113.793423 92) (width 0.25) (layer "B.Cu") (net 2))
 (segment (start 66.793423 89.2755) (end 66.793423 94.2755) (width 0.25) (layer "F.Cu") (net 5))
 (segment (start 63.068923 98) (end 62.793423 98) (width 0.25) (layer "F.Cu") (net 5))
 (segment (start 66.793423 94.2755) (end 63.068923 98) (width 0.25) (layer "F.Cu") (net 5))
 (segment (start 66.793423 98) (end 62.793423 98) (width 0.25) (layer "F.Cu") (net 5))
 (via (at 66.793423 98) (size 0.8) (drill 0.4) (layers "F.Cu" "B.Cu") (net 5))
 (via (at 66.793423 89.2755) (size 0.8) (drill 0.4) (layers "F.Cu" "B.Cu") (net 5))
 (segment (start 159.343423 91.55) (end 186.243423 91.55) (width 0.25) (layer "B.Cu") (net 5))
 (segment (start 77.705319 89.2755) (end 80.429819 92) (width 0.25) (layer "B.Cu") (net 5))
 (segment (start 187.173423 90.62) (end 187.173423 89.76) (width 0.25) (layer "B.Cu") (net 5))
 (segment (start 186.243423 91.55) (end 187.173423 90.62) (width 0.25) (layer "B.Cu") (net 5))
 (segment (start 117.793423 87) (end 154.793423 87) (width 0.25) (layer "B.Cu") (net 5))
 (segment (start 83.263025 91.55) (end 113.243423 91.55) (width 0.25) (layer "B.Cu") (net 5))
 (segment (start 113.243423 91.55) (end 117.793423 87) (width 0.25) (layer "B.Cu") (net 5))
 (segment (start 154.793423 87) (end 159.343423 91.55) (width 0.25) (layer "B.Cu") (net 5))
 (segment (start 80.429819 92) (end 82.813025 92) (width 0.25) (layer "B.Cu") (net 5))
 (segment (start 66.871423 98.078) (end 66.793423 98) (width 0.25) (layer "B.Cu") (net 5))
 (segment (start 66.793423 89.2755) (end 77.705319 89.2755) (width 0.25) (layer "B.Cu") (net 5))
 (segment (start 82.813025 92) (end 83.263025 91.55) (width 0.25) (layer "B.Cu") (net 5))
 (segment (start 72.793423 98.078) (end 66.871423 98.078) (width 0.25) (layer "B.Cu") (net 5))
 (segment (start 103.793423 99.871072) (end 104.189959 99.474536) (width 0.25) (layer "F.Cu") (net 10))
 (segment (start 103.793423 103) (end 103.793423 99.871072) (width 0.25) (layer "F.Cu") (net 10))
 (via (at 102.793423 93.2755) (size 0.8) (drill 0.4) (layers "F.Cu" "B.Cu") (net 10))
 (segment (start 116.793423 95) (end 115.793423 94) (width 0.25) (layer "B.Cu") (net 10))
 (segment (start 188.793423 95) (end 116.793423 95) (width 0.25) (layer "B.Cu") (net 10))
 (segment (start 103.517923 94) (end 102.793423 93.2755) (width 0.25) (layer "B.Cu") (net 10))
 (segment (start 192.253423 89.76) (end 192.253423 91.54) (width 0.25) (layer "B.Cu") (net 10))
 (segment (start 115.793423 94) (end 103.517923 94) (width 0.25) (layer "B.Cu") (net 10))
 (segment (start 192.253423 91.54) (end 188.793423 95) (width 0.25) (layer "B.Cu") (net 10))
 (segment (start 113.793423 87) (end 111.793423 85) (width 0.25) (layer "F.Cu") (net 7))
 (segment (start 102.333423 85) (end 100.333423 87) (width 0.25) (layer "F.Cu") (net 7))
 (segment (start 113.793423 95) (end 113.793423 87) (width 0.25) (layer "F.Cu") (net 7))
 (segment (start 111.793423 85) (end 102.333423 85) (width 0.25) (layer "F.Cu") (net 7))
 (via (at 113.793423 95) (size 0.8) (drill 0.4) (layers "F.Cu" "B.Cu") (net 7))
 (segment (start 113.793423 95) (end 115.793423 95) (width 0.25) (layer "B.Cu") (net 7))
 (segment (start 115.793423 95) (end 116.343423 95.55) (width 0.25) (layer "B.Cu") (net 7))
 (segment (start 116.343423 95.55) (end 191.243423 95.55) (width 0.25) (layer "B.Cu") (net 7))
 (segment (start 191.243423 95.55) (end 194.793423 92) (width 0.25) (layer "B.Cu") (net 7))
 (segment (start 194.793423 92) (end 194.793423 89.76) (width 0.25) (layer "B.Cu") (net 7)))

